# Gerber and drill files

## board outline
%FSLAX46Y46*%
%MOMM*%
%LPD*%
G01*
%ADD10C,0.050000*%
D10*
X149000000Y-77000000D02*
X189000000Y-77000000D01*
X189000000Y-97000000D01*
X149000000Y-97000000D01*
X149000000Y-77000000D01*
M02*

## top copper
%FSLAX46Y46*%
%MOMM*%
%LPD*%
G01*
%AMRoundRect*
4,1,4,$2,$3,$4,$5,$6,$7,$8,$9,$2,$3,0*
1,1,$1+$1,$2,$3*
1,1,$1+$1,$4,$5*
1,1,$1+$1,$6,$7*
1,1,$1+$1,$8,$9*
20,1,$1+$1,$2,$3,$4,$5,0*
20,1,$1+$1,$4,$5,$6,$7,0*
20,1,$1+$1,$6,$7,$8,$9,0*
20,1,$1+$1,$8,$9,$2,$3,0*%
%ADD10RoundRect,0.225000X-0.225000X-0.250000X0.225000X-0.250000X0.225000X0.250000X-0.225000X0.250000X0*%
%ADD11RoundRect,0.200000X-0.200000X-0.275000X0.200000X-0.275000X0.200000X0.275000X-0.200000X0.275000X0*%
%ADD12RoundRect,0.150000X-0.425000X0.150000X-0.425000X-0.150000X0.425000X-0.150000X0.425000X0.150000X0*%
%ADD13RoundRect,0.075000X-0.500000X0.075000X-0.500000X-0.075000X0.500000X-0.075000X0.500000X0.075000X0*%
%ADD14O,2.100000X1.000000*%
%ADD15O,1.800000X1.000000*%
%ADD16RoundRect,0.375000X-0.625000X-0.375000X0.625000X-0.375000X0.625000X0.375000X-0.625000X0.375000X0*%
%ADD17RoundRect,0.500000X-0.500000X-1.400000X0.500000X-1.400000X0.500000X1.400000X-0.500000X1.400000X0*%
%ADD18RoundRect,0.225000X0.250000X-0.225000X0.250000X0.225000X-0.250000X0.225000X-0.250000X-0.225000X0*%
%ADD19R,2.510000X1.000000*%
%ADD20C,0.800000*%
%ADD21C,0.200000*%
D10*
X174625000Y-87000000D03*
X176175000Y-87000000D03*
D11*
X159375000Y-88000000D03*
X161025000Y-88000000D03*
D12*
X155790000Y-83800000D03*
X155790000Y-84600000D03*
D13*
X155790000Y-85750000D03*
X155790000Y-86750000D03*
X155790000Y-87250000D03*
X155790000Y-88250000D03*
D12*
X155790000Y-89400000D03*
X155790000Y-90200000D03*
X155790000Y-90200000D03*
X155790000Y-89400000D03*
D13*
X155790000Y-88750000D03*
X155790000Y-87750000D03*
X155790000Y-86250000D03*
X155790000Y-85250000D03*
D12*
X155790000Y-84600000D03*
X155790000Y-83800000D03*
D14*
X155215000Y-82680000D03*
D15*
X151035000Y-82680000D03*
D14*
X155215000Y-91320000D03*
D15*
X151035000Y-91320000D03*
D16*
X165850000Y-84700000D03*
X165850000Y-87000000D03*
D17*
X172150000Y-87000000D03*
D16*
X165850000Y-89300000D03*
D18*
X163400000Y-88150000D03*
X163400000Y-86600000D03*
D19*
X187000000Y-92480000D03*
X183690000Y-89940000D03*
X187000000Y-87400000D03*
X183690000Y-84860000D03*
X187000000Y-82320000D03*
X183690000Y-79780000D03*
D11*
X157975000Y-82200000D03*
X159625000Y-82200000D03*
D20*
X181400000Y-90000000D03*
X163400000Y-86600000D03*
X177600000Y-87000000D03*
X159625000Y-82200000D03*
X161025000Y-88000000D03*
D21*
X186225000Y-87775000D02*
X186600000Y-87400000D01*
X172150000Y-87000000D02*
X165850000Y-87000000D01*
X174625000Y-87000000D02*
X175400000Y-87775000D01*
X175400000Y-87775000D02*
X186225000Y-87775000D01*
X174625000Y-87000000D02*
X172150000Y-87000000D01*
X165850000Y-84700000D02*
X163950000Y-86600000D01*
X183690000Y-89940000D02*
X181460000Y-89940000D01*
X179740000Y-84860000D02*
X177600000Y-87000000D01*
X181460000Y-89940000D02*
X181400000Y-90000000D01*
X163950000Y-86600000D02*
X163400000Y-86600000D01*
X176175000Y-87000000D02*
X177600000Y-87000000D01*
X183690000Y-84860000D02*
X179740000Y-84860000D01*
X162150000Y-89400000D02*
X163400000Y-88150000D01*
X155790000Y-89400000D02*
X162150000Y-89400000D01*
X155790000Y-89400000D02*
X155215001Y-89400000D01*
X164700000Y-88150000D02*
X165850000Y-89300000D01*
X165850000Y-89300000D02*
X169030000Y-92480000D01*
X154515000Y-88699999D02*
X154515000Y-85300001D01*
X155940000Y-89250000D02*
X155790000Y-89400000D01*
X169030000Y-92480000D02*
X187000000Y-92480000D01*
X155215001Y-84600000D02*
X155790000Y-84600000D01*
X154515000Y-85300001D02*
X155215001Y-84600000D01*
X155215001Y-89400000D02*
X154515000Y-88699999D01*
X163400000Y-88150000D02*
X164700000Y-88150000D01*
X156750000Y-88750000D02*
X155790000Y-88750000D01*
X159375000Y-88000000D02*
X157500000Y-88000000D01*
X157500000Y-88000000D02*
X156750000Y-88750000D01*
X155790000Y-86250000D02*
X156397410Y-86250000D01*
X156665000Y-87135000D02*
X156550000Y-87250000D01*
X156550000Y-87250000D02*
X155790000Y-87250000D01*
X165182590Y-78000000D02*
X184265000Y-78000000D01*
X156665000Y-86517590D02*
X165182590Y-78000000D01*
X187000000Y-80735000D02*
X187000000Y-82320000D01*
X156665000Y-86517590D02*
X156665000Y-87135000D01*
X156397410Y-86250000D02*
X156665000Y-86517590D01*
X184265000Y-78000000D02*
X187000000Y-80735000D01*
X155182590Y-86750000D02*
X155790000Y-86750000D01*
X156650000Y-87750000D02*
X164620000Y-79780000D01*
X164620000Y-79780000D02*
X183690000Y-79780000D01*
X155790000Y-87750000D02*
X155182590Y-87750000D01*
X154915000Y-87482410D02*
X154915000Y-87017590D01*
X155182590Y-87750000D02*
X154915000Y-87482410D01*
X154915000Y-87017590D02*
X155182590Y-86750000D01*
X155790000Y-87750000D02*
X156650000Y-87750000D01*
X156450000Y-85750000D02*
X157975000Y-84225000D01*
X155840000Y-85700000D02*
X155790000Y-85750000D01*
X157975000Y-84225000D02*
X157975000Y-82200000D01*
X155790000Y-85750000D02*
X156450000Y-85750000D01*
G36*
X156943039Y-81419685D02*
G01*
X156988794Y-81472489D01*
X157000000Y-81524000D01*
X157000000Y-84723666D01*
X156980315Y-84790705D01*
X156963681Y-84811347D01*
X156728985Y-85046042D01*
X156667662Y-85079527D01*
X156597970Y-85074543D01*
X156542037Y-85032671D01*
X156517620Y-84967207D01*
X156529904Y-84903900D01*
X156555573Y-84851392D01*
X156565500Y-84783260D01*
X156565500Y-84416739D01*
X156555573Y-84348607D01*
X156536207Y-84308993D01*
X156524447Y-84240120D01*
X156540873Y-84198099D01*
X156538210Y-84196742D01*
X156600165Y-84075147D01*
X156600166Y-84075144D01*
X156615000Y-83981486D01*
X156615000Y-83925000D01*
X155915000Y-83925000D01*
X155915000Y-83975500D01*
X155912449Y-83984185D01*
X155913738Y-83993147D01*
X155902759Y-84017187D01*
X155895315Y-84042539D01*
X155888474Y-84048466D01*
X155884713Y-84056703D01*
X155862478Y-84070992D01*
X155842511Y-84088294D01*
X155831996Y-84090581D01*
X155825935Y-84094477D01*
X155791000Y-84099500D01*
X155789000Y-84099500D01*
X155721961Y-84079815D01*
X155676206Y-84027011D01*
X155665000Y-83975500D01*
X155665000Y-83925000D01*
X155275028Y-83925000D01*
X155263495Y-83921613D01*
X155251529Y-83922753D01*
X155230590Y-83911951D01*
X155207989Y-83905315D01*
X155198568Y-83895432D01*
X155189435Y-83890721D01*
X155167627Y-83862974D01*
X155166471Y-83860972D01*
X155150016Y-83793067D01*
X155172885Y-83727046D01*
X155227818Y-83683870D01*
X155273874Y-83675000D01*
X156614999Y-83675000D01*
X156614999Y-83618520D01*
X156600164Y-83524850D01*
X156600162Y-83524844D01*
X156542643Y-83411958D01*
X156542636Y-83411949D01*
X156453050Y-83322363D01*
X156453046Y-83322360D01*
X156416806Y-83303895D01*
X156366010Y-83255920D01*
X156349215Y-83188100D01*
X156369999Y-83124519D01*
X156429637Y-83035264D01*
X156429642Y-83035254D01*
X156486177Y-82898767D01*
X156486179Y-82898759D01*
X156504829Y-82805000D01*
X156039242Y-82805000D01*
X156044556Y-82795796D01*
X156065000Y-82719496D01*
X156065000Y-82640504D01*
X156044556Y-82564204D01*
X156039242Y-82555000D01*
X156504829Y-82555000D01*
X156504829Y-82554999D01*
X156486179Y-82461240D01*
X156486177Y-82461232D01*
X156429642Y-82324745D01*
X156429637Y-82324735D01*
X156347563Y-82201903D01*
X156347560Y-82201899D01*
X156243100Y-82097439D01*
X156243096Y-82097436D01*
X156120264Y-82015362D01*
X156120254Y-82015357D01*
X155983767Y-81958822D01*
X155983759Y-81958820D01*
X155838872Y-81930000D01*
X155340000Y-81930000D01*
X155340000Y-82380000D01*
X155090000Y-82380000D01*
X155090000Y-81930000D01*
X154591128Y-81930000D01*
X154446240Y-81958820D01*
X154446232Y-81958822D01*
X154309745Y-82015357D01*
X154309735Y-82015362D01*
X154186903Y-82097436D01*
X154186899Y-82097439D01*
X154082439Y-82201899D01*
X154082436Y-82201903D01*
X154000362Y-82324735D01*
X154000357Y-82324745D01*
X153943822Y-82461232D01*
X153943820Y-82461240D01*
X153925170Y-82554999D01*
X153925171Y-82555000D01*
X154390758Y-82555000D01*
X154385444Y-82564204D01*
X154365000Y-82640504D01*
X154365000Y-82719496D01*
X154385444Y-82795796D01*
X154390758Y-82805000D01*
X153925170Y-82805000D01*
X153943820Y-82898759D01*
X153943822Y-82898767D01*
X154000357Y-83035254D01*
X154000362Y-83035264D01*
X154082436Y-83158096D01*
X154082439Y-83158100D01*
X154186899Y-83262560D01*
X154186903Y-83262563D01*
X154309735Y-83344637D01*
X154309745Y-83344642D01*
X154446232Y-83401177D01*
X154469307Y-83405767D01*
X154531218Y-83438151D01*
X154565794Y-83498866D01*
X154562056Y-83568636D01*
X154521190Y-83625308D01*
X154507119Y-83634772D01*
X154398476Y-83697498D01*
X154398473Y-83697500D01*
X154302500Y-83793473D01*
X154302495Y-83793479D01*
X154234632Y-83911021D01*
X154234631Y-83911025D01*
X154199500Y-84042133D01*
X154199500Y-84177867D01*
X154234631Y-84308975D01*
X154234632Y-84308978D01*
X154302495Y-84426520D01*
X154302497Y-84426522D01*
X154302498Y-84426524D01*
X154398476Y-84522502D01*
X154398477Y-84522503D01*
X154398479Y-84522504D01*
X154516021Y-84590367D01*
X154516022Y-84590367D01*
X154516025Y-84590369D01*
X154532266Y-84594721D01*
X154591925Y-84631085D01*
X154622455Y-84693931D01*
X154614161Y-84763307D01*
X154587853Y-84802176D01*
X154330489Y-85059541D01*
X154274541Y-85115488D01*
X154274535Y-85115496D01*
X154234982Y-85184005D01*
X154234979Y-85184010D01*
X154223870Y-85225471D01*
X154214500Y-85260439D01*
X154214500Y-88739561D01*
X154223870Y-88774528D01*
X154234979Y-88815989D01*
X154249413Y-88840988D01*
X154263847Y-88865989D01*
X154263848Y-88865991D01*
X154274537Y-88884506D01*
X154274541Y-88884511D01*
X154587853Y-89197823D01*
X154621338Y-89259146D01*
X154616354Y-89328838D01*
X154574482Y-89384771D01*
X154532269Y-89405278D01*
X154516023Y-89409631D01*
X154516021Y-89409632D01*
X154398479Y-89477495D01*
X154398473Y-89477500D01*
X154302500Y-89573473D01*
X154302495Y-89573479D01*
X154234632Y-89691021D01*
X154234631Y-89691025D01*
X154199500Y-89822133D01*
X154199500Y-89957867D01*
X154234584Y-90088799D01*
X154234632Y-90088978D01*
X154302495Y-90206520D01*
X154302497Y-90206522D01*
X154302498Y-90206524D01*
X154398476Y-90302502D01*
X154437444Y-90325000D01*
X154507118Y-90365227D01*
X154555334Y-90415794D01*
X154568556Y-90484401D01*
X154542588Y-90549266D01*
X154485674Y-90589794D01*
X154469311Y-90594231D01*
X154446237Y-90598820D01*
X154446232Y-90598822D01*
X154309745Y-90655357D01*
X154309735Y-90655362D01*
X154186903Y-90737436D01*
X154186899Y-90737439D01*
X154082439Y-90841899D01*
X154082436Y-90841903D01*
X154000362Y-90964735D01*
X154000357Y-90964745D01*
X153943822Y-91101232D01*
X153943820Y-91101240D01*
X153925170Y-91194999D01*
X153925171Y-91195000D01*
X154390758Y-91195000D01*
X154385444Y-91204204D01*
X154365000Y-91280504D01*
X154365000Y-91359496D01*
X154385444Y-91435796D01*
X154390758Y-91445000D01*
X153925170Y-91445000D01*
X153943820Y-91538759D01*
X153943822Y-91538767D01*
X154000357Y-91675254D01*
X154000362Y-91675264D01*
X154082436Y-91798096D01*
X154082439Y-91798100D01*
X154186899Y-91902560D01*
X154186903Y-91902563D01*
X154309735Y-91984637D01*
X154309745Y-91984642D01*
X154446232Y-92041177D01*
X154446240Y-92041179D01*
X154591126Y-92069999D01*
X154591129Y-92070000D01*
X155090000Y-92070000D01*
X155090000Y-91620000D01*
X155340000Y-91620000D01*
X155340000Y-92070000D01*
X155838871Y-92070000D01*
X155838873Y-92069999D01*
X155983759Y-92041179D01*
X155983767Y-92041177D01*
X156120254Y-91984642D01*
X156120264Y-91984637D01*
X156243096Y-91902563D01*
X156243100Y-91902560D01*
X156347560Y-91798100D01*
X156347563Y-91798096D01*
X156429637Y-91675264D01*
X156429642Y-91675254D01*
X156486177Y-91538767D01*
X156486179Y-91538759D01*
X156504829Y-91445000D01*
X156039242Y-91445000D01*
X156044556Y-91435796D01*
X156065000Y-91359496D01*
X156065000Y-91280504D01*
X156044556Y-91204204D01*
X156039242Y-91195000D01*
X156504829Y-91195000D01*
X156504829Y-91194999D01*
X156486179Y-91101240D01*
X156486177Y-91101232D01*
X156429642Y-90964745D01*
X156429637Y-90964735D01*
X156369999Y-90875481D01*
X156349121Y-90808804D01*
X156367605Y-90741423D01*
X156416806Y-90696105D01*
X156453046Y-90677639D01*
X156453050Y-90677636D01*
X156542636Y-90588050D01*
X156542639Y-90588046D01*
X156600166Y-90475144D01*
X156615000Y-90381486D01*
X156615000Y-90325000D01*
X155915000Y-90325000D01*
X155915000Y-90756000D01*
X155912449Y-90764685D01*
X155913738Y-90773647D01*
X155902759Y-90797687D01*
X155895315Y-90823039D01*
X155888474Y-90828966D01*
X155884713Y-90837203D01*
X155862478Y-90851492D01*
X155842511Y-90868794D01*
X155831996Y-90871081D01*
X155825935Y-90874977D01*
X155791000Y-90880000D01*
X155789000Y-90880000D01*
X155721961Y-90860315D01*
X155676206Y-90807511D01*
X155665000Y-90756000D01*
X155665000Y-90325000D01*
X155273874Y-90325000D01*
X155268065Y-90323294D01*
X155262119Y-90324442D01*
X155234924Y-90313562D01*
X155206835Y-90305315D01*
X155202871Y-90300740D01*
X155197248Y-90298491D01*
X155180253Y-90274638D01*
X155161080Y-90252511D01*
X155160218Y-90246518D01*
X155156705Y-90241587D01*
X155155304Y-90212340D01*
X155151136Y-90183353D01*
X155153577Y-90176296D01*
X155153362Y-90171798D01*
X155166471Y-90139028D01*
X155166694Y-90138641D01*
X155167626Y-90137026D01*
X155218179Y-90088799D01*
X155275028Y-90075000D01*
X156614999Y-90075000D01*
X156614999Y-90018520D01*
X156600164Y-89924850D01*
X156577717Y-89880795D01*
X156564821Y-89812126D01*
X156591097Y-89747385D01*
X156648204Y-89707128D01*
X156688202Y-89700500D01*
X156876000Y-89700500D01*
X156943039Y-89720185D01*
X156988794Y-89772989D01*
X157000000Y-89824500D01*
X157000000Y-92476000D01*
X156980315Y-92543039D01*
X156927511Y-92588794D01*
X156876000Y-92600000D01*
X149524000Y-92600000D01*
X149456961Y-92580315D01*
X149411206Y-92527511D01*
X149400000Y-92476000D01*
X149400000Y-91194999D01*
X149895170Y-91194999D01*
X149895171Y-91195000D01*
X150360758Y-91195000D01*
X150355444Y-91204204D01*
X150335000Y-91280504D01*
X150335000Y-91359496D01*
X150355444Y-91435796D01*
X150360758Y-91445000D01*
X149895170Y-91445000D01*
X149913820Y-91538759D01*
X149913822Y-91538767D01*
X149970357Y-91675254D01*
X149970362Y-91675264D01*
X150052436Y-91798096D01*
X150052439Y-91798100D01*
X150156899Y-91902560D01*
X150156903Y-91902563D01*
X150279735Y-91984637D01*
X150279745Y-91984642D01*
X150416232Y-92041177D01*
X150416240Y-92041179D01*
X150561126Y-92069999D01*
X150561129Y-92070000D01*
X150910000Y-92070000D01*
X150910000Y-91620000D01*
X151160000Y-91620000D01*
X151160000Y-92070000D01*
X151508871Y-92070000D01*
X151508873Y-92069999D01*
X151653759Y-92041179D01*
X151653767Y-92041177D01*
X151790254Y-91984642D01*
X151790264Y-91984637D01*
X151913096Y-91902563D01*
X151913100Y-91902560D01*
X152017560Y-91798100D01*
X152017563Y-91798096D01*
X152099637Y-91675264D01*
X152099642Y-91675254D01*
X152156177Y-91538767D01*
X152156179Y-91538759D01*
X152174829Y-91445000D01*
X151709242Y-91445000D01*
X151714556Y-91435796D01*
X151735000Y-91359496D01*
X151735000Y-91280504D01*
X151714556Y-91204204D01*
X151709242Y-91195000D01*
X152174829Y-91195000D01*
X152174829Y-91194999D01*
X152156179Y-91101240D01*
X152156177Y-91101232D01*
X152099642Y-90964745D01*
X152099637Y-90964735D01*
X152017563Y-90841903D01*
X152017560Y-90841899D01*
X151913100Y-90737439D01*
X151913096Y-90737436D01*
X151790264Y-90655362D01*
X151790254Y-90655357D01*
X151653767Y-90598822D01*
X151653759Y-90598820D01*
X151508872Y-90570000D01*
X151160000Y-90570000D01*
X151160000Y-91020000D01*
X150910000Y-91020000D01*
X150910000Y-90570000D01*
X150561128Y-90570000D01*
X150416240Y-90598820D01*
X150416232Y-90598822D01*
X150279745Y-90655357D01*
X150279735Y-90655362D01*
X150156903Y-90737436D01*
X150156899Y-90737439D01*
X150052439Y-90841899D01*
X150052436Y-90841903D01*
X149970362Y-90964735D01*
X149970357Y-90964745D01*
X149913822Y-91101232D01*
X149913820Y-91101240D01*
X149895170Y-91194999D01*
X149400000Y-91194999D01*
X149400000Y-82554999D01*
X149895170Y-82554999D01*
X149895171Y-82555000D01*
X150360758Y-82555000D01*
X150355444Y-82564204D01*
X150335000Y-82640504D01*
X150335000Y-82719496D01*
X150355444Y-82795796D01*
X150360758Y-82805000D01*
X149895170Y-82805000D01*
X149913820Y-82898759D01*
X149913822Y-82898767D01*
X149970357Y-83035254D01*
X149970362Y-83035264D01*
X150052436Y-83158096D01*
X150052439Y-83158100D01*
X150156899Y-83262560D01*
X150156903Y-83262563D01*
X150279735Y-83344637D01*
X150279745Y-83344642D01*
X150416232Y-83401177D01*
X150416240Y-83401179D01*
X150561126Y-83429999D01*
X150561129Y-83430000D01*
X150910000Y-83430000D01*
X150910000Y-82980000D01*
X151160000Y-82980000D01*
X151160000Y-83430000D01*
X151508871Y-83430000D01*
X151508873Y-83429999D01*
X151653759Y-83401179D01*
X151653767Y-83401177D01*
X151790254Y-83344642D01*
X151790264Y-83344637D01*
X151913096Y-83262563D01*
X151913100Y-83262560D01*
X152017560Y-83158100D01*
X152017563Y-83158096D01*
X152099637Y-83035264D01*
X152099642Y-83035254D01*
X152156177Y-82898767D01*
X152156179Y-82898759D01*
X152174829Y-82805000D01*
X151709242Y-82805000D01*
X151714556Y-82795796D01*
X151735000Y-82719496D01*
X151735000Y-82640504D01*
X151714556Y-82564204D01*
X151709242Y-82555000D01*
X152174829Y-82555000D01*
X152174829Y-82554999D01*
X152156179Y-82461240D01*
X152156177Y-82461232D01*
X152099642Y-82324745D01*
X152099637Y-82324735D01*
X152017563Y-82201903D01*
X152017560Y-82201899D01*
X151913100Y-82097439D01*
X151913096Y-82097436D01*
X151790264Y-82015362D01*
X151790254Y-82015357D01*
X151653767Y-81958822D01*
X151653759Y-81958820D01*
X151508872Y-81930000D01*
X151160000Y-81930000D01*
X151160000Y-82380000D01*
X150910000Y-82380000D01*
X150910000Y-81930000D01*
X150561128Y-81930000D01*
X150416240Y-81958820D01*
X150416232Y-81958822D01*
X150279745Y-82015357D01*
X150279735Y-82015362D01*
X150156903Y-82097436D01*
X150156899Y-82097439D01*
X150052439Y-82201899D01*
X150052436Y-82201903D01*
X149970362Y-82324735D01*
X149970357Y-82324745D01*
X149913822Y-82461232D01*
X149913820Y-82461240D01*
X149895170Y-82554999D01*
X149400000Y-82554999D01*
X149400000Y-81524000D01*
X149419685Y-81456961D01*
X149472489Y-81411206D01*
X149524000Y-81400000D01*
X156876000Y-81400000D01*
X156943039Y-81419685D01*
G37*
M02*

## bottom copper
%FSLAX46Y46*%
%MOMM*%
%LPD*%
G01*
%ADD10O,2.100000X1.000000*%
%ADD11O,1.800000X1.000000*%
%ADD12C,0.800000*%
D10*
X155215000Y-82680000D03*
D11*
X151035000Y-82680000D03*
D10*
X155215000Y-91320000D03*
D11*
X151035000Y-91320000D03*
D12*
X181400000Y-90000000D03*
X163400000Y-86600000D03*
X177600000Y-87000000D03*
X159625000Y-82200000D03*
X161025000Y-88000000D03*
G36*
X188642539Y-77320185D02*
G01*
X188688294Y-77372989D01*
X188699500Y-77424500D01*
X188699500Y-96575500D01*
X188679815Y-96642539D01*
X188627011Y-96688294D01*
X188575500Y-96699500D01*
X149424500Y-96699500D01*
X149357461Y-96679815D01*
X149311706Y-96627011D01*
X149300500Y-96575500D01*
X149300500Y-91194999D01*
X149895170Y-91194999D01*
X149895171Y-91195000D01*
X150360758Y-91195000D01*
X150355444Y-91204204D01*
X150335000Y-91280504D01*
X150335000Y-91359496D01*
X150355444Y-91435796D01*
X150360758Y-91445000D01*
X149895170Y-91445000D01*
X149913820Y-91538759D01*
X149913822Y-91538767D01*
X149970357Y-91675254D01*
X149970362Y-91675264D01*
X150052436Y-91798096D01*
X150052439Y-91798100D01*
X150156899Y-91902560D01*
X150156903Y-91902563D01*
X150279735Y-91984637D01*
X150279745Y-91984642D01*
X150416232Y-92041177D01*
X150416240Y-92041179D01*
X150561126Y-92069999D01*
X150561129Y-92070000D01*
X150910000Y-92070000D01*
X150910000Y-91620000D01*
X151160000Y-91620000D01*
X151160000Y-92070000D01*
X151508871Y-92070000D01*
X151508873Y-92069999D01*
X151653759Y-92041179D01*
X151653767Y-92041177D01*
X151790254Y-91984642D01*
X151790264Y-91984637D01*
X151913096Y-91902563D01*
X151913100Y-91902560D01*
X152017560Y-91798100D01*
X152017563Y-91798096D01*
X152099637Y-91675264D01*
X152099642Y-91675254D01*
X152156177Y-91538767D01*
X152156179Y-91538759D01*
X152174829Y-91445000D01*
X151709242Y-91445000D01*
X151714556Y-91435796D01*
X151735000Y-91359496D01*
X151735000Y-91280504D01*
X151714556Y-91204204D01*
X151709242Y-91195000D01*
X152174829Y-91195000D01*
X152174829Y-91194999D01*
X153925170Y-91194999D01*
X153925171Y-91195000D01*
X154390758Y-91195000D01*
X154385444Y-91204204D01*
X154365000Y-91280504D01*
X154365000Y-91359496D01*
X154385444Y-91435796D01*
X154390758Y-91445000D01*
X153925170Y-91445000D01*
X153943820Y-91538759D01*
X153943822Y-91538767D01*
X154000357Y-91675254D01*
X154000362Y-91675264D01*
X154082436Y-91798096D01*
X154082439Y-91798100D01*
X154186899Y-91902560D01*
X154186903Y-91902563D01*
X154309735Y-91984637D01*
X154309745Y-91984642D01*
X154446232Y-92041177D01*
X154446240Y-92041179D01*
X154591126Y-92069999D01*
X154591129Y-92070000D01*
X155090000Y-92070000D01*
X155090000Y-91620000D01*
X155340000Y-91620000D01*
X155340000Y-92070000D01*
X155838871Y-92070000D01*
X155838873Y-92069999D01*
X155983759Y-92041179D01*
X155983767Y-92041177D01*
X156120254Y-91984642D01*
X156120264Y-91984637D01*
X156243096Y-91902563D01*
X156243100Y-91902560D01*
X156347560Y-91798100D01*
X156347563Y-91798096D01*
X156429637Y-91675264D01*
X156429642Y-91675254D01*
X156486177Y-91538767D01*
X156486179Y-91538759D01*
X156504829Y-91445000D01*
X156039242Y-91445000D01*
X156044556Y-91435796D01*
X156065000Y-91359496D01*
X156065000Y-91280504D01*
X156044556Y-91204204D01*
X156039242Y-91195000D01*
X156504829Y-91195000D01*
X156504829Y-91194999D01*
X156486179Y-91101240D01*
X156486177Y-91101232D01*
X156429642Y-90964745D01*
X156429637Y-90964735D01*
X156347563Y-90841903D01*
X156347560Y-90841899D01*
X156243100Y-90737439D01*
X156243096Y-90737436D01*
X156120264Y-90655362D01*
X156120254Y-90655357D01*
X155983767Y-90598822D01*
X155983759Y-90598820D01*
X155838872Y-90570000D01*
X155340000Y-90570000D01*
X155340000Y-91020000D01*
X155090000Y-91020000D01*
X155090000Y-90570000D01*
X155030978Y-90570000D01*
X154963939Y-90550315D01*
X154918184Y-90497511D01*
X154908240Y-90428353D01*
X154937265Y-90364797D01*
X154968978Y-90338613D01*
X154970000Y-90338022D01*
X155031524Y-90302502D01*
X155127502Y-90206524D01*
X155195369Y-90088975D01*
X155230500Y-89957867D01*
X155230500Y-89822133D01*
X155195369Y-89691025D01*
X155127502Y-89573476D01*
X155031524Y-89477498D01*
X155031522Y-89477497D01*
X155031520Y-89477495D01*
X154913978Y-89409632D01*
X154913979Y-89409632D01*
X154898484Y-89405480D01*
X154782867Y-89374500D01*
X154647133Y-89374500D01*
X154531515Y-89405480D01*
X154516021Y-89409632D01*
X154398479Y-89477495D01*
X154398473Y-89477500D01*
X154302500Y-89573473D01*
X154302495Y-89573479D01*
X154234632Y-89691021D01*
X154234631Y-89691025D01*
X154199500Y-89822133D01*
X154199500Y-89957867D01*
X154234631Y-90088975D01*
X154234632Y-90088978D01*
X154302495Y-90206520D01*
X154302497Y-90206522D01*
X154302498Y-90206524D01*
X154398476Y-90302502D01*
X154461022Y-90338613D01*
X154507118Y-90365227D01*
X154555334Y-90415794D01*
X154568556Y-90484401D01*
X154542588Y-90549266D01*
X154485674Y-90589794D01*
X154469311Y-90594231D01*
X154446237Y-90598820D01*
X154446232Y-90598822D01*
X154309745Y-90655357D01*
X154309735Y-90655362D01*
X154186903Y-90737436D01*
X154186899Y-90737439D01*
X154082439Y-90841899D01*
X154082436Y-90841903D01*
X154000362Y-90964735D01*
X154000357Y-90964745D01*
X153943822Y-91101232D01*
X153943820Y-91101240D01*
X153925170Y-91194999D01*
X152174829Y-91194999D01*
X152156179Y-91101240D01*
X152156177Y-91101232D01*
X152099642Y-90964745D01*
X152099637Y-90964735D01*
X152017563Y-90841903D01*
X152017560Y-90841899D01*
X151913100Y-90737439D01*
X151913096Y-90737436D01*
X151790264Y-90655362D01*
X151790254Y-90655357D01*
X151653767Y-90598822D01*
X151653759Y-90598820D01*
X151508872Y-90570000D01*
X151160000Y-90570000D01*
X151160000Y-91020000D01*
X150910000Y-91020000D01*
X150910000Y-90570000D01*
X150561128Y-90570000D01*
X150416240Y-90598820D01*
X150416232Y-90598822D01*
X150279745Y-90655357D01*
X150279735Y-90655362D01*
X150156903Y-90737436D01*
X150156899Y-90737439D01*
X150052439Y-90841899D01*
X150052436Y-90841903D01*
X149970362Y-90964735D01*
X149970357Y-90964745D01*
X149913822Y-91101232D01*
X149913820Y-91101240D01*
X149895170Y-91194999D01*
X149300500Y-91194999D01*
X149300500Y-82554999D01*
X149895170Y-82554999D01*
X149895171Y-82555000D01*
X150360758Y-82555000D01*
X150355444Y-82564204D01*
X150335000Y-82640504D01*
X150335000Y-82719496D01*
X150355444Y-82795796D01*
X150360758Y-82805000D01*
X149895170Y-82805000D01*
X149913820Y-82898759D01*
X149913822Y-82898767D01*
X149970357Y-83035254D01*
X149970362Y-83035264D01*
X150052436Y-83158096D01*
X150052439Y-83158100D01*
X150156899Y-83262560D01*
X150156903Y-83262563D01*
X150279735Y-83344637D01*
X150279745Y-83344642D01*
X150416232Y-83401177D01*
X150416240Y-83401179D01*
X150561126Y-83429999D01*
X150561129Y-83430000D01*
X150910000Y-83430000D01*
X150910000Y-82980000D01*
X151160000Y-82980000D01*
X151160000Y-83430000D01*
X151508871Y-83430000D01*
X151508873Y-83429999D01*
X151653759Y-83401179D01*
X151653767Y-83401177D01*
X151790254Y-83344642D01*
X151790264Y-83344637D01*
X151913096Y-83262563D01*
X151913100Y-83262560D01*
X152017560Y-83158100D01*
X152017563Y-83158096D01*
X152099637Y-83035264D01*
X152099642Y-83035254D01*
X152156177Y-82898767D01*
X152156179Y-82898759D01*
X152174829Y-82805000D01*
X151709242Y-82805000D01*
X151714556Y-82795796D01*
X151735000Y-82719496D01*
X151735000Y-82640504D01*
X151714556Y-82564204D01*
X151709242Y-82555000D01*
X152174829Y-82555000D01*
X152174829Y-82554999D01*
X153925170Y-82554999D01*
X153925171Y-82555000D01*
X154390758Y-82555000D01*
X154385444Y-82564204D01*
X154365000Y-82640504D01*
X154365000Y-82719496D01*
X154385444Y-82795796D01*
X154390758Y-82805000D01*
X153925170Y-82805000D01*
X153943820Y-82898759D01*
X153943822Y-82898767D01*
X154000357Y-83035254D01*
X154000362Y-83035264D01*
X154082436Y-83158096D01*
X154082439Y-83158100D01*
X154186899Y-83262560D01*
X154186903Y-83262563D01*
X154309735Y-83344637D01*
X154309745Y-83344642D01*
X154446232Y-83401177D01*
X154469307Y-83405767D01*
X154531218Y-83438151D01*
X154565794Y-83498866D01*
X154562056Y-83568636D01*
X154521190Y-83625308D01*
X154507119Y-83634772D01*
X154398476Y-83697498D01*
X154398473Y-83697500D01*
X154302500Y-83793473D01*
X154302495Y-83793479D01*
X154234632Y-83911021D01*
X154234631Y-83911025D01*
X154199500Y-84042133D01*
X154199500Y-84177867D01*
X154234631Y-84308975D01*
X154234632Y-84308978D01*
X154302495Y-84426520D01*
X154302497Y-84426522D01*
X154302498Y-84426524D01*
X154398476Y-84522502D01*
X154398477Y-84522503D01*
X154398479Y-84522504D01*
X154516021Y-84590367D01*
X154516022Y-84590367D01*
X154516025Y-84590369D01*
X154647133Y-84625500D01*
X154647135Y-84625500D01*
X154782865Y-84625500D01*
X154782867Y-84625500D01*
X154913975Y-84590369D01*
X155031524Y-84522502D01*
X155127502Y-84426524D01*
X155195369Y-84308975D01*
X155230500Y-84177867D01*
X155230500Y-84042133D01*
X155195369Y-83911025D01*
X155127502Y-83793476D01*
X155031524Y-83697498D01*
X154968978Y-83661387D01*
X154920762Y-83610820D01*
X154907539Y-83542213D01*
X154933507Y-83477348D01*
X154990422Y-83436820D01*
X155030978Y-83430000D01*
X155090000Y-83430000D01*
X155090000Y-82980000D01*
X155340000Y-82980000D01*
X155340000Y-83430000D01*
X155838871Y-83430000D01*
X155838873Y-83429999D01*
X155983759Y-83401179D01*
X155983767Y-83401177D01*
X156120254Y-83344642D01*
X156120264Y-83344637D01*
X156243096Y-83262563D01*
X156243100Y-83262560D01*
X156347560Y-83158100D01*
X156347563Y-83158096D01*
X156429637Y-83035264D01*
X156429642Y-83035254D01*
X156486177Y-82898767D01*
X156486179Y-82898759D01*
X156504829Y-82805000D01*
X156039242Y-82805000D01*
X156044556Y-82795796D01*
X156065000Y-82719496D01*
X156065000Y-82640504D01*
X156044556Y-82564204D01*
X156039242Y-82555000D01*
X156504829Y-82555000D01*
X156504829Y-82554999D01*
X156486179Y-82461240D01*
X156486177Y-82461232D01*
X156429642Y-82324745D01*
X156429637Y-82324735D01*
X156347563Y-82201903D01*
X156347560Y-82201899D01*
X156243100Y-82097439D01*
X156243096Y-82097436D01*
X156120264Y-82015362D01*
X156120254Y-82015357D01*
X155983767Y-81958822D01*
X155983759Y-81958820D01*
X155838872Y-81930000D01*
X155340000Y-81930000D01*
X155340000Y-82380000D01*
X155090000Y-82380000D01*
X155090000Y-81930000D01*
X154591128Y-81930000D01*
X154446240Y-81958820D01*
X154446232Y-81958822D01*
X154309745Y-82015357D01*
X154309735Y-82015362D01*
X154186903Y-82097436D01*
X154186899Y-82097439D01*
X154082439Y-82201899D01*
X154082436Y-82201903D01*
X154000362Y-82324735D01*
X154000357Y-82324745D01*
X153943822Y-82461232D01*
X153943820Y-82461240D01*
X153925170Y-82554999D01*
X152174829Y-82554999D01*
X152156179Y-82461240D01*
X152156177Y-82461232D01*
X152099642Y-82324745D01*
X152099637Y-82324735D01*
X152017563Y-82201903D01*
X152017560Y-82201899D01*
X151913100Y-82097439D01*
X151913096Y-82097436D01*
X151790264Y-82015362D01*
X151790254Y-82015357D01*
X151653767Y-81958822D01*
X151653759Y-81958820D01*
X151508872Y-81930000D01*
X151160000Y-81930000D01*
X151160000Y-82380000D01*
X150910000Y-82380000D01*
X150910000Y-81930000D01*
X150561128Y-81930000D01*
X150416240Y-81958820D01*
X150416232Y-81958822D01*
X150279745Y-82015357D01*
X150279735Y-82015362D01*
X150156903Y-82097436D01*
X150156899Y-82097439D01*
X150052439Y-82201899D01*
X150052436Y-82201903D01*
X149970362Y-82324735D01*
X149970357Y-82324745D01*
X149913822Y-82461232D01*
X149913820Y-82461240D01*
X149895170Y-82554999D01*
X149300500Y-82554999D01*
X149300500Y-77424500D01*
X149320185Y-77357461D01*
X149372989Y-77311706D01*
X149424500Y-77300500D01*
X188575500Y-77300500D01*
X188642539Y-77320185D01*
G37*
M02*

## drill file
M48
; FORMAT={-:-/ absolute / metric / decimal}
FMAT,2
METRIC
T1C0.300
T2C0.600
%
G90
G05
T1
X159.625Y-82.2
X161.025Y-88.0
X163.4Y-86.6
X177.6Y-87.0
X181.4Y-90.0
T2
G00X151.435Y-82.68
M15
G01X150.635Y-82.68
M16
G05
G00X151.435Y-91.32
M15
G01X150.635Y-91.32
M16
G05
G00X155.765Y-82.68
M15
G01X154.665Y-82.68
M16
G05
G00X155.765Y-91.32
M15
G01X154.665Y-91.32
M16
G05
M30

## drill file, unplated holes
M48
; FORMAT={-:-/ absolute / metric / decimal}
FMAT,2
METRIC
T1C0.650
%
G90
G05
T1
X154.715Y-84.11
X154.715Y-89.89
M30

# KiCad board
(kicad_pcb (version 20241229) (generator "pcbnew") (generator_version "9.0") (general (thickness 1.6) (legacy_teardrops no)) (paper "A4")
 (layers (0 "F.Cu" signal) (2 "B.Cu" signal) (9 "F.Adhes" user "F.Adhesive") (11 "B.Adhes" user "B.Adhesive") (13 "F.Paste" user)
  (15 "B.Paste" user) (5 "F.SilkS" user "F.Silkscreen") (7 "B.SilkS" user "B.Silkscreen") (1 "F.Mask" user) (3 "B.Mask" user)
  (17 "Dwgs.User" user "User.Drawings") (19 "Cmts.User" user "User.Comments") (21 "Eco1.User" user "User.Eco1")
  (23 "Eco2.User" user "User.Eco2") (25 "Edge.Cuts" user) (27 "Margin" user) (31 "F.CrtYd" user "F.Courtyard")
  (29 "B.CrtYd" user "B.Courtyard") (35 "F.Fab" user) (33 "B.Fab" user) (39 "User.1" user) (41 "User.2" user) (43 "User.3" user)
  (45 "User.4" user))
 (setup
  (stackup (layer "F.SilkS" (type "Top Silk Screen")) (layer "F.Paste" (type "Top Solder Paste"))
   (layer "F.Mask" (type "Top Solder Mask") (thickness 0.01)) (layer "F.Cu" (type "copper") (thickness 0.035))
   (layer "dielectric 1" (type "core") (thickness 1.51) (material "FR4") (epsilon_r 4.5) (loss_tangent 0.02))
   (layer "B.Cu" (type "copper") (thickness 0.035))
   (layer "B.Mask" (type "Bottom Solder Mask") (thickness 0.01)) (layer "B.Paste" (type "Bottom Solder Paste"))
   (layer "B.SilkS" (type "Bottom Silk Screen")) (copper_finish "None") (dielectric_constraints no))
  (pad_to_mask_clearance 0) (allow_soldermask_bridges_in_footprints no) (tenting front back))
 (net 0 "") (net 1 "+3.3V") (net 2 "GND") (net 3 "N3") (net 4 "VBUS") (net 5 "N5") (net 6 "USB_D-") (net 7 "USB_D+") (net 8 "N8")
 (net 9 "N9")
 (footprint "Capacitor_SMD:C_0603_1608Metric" (layer "F.Cu") (at 175.4 87)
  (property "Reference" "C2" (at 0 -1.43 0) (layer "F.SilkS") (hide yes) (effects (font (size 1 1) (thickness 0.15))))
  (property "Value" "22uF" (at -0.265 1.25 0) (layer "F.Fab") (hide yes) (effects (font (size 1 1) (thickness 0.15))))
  (pad "1" smd roundrect (at -0.775 0) (size 0.9 0.95) (layers "F.Cu" "F.Mask" "F.Paste") (roundrect_rratio 0.25) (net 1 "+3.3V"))
  (pad "2" smd roundrect (at 0.775 0) (size 0.9 0.95) (layers "F.Cu" "F.Mask" "F.Paste") (roundrect_rratio 0.25) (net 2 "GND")))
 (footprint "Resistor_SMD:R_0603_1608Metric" (layer "F.Cu") (at 160.2 88)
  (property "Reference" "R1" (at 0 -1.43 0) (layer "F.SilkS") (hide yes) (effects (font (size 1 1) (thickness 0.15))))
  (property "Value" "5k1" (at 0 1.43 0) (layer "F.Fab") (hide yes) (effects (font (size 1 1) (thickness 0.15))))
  (pad "1" smd roundrect (at -0.825 0) (size 0.8 0.95) (layers "F.Cu" "F.Mask" "F.Paste") (roundrect_rratio 0.25) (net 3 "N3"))
  (pad "2" smd roundrect (at 0.825 0) (size 0.8 0.95) (layers "F.Cu" "F.Mask" "F.Paste") (roundrect_rratio 0.25) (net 2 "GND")))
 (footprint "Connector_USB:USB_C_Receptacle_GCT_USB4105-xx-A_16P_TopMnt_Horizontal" (layer "F.Cu") (at 152.11 87 -90)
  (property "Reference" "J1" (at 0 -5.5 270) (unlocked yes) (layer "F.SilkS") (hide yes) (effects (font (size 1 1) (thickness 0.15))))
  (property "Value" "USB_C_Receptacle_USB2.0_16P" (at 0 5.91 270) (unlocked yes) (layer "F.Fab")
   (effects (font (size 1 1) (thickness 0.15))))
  (pad "" np_thru_hole circle (at -2.89 -2.605 270) (size 0.65 0.65) (drill 0.65) (layers "*.Cu" "*.Mask"))
  (pad "" np_thru_hole circle (at 2.89 -2.605 270) (size 0.65 0.65) (drill 0.65) (layers "*.Cu" "*.Mask"))
  (pad "A1" smd roundrect (at -3.2 -3.68 270) (size 0.6 1.15) (layers "F.Cu" "F.Mask" "F.Paste") (roundrect_rratio 0.25) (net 2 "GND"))
  (pad "A4" smd roundrect (at -2.4 -3.68 270) (size 0.6 1.15) (layers "F.Cu" "F.Mask" "F.Paste") (roundrect_rratio 0.25) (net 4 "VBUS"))
  (pad "A5" smd roundrect (at -1.25 -3.68 270) (size 0.3 1.15) (layers "F.Cu" "F.Mask" "F.Paste") (roundrect_rratio 0.25) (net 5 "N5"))
  (pad "A6" smd roundrect (at -0.25 -3.68 270) (size 0.3 1.15) (layers "F.Cu" "F.Mask" "F.Paste") (roundrect_rratio 0.25) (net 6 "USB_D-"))
  (pad "A7" smd roundrect (at 0.25 -3.68 270) (size 0.3 1.15) (layers "F.Cu" "F.Mask" "F.Paste") (roundrect_rratio 0.25) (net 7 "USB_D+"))
  (pad "A8" smd roundrect (at 1.25 -3.68 270) (size 0.3 1.15) (layers "F.Cu" "F.Mask" "F.Paste") (roundrect_rratio 0.25) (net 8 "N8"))
  (pad "A9" smd roundrect (at 2.4 -3.68 270) (size 0.6 1.15) (layers "F.Cu" "F.Mask" "F.Paste") (roundrect_rratio 0.25) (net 4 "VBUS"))
  (pad "A12" smd roundrect (at 3.2 -3.68 270) (size 0.6 1.15) (layers "F.Cu" "F.Mask" "F.Paste") (roundrect_rratio 0.25) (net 2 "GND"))
  (pad "B1" smd roundrect (at 3.2 -3.68 270) (size 0.6 1.15) (layers "F.Cu" "F.Mask" "F.Paste") (roundrect_rratio 0.25) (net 2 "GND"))
  (pad "B4" smd roundrect (at 2.4 -3.68 270) (size 0.6 1.15) (layers "F.Cu" "F.Mask" "F.Paste") (roundrect_rratio 0.25) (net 4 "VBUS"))
  (pad "B5" smd roundrect (at 1.75 -3.68 270) (size 0.3 1.15) (layers "F.Cu" "F.Mask" "F.Paste") (roundrect_rratio 0.25) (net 3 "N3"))
  (pad "B6" smd roundrect (at 0.75 -3.68 270) (size 0.3 1.15) (layers "F.Cu" "F.Mask" "F.Paste") (roundrect_rratio 0.25) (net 6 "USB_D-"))
  (pad "B7" smd roundrect (at -0.75 -3.68 270) (size 0.3 1.15) (layers "F.Cu" "F.Mask" "F.Paste") (roundrect_rratio 0.25) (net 7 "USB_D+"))
  (pad "B8" smd roundrect (at -1.75 -3.68 270) (size 0.3 1.15) (layers "F.Cu" "F.Mask" "F.Paste") (roundrect_rratio 0.25) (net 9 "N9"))
  (pad "B9" smd roundrect (at -2.4 -3.68 270) (size 0.6 1.15) (layers "F.Cu" "F.Mask" "F.Paste") (roundrect_rratio 0.25) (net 4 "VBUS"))
  (pad "B12" smd roundrect (at -3.2 -3.68 270) (size 0.6 1.15) (layers "F.Cu" "F.Mask" "F.Paste") (roundrect_rratio 0.25) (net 2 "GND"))
  (pad "S1" thru_hole oval (at -4.32 -3.105 270) (size 1 2.1) (drill oval 0.6 1.7) (layers "*.Cu" "*.Mask" "F.Paste")
   (remove_unused_layers no) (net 2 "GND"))
  (pad "S1" thru_hole oval (at -4.32 1.075 270) (size 1 1.8) (drill oval 0.6 1.4) (layers "*.Cu" "*.Mask" "F.Paste")
   (remove_unused_layers no) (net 2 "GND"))
  (pad "S1" thru_hole oval (at 4.32 -3.105 270) (size 1 2.1) (drill oval 0.6 1.7) (layers "*.Cu" "*.Mask" "F.Paste")
   (remove_unused_layers no) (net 2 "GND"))
  (pad "S1" thru_hole oval (at 4.32 1.075 270) (size 1 1.8) (drill oval 0.6 1.4) (layers "*.Cu" "*.Mask" "F.Paste")
   (remove_unused_layers no) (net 2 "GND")))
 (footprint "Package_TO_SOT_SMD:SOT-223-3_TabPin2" (layer "F.Cu") (at 169 87)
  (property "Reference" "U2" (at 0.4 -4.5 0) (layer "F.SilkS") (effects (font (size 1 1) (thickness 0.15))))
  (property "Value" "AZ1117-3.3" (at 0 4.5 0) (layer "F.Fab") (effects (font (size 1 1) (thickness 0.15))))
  (pad "1" smd roundrect (at -3.15 -2.3) (size 2 1.5) (layers "F.Cu" "F.Mask" "F.Paste") (roundrect_rratio 0.25) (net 2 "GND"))
  (pad "2" smd roundrect (at -3.15 0) (size 2 1.5) (layers "F.Cu" "F.Mask" "F.Paste") (roundrect_rratio 0.25) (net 1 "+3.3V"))
  (pad "2" smd roundrect (at 3.15 0) (size 2 3.8) (layers "F.Cu" "F.Mask" "F.Paste") (roundrect_rratio 0.25) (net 1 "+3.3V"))
  (pad "3" smd roundrect (at -3.15 2.3) (size 2 1.5) (layers "F.Cu" "F.Mask" "F.Paste") (roundrect_rratio 0.25) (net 4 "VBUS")))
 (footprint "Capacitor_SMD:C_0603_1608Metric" (layer "F.Cu") (at 163.4 87.375 90)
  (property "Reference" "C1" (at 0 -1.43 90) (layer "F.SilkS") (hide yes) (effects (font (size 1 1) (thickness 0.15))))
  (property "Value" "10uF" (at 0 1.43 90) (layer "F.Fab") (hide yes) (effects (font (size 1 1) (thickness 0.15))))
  (pad "1" smd roundrect (at -0.775 0 90) (size 0.9 0.95) (layers "F.Cu" "F.Mask" "F.Paste") (roundrect_rratio 0.25) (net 4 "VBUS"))
  (pad "2" smd roundrect (at 0.775 0 90) (size 0.9 0.95) (layers "F.Cu" "F.Mask" "F.Paste") (roundrect_rratio 0.25) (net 2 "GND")))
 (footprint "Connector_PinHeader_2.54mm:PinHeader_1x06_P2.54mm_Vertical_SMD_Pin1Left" (layer "F.Cu") (at 185.345 86.13 180)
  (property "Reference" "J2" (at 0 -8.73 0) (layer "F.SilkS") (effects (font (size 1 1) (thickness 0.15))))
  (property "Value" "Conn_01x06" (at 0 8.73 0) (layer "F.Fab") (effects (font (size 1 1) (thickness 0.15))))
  (pad "1" smd rect (at -1.655 -6.35 180) (size 2.51 1) (layers "F.Cu" "F.Mask" "F.Paste") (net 4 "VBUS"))
  (pad "2" smd rect (at 1.655 -3.81 180) (size 2.51 1) (layers "F.Cu" "F.Mask" "F.Paste") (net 2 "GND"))
  (pad "3" smd rect (at -1.655 -1.27 180) (size 2.51 1) (layers "F.Cu" "F.Mask" "F.Paste") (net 1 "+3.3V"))
  (pad "4" smd rect (at 1.655 1.27 180) (size 2.51 1) (layers "F.Cu" "F.Mask" "F.Paste") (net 2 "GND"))
  (pad "5" smd rect (at -1.655 3.81 180) (size 2.51 1) (layers "F.Cu" "F.Mask" "F.Paste") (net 7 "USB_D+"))
  (pad "6" smd rect (at 1.655 6.35 180) (size 2.51 1) (layers "F.Cu" "F.Mask" "F.Paste") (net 6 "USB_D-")))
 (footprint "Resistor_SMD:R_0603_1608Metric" (layer "F.Cu") (at 158.8 82.2)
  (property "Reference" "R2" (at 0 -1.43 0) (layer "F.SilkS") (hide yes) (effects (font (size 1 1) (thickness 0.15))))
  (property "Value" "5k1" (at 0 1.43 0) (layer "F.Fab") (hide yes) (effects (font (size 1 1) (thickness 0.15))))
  (pad "1" smd roundrect (at -0.825 0) (size 0.8 0.95) (layers "F.Cu" "F.Mask" "F.Paste") (roundrect_rratio 0.25) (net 5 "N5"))
  (pad "2" smd roundrect (at 0.825 0) (size 0.8 0.95) (layers "F.Cu" "F.Mask" "F.Paste") (roundrect_rratio 0.25) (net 2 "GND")))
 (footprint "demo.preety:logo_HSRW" (layer "F.Cu") (at 161.4 94)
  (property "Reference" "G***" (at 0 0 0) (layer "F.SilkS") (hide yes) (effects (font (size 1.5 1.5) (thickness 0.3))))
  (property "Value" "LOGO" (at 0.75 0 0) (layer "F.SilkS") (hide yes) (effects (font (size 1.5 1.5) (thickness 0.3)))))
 (gr_rect (start 149 77) (end 189 97) (stroke (width 0.05) (type default)) (fill no) (layer "Edge.Cuts"))
 (segment (start 186.225 87.775) (end 186.6 87.4) (width 0.2) (layer "F.Cu") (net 1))
 (segment (start 172.15 87) (end 165.85 87) (width 0.2) (layer "F.Cu") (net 1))
 (segment (start 174.625 87) (end 175.4 87.775) (width 0.2) (layer "F.Cu") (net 1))
 (segment (start 175.4 87.775) (end 186.225 87.775) (width 0.2) (layer "F.Cu") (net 1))
 (segment (start 174.625 87) (end 172.15 87) (width 0.2) (layer "F.Cu") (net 1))
 (segment (start 165.85 84.7) (end 163.95 86.6) (width 0.2) (layer "F.Cu") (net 2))
 (segment (start 183.69 89.94) (end 181.46 89.94) (width 0.2) (layer "F.Cu") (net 2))
 (segment (start 179.74 84.86) (end 177.6 87) (width 0.2) (layer "F.Cu") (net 2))
 (segment (start 181.46 89.94) (end 181.4 90) (width 0.2) (layer "F.Cu") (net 2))
 (segment (start 163.95 86.6) (end 163.4 86.6) (width 0.2) (layer "F.Cu") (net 2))
 (segment (start 176.175 87) (end 177.6 87) (width 0.2) (layer "F.Cu") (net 2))
 (segment (start 183.69 84.86) (end 179.74 84.86) (width 0.2) (layer "F.Cu") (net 2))
 (via (at 181.4 90) (size 0.8) (drill 0.3) (layers "F.Cu" "B.Cu") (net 2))
 (via (at 163.4 86.6) (size 0.8) (drill 0.3) (layers "F.Cu" "B.Cu") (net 2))
 (via (at 177.6 87) (size 0.8) (drill 0.3) (layers "F.Cu" "B.Cu") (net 2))
 (via (at 159.625 82.2) (size 0.8) (drill 0.3) (layers "F.Cu" "B.Cu") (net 2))
 (via (at 161.025 88) (size 0.8) (drill 0.3) (layers "F.Cu" "B.Cu") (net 2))
 (segment (start 162.15 89.4) (end 163.4 88.15) (width 0.2) (layer "F.Cu") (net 4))
 (segment (start 155.79 89.4) (end 162.15 89.4) (width 0.2) (layer "F.Cu") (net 4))
 (segment (start 155.79 89.4) (end 155.215001 89.4) (width 0.2) (layer "F.Cu") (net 4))
 (segment (start 164.7 88.15) (end 165.85 89.3) (width 0.2) (layer "F.Cu") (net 4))
 (segment (start 165.85 89.3) (end 169.03 92.48) (width 0.2) (layer "F.Cu") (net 4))
 (segment (start 154.515 88.699999) (end 154.515 85.300001) (width 0.2) (layer "F.Cu") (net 4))
 (segment (start 155.94 89.25) (end 155.79 89.4) (width 0.2) (layer "F.Cu") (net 4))
 (segment (start 169.03 92.48) (end 187 92.48) (width 0.2) (layer "F.Cu") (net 4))
 (segment (start 155.215001 84.6) (end 155.79 84.6) (width 0.2) (layer "F.Cu") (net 4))
 (segment (start 154.515 85.300001) (end 155.215001 84.6) (width 0.2) (layer "F.Cu") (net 4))
 (segment (start 155.215001 89.4) (end 154.515 88.699999) (width 0.2) (layer "F.Cu") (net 4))
 (segment (start 163.4 88.15) (end 164.7 88.15) (width 0.2) (layer "F.Cu") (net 4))
 (segment (start 156.75 88.75) (end 155.79 88.75) (width 0.2) (layer "F.Cu") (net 3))
 (segment (start 159.375 88) (end 157.5 88) (width 0.2) (layer "F.Cu") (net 3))
 (segment (start 157.5 88) (end 156.75 88.75) (width 0.2) (layer "F.Cu") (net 3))
 (segment (start 155.79 86.25) (end 156.39741 86.25) (width 0.2) (layer "F.Cu") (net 7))
 (segment (start 156.665 87.135) (end 156.55 87.25) (width 0.2) (layer "F.Cu") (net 7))
 (segment (start 156.55 87.25) (end 155.79 87.25) (width 0.2) (layer "F.Cu") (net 7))
 (segment (start 165.18259 78) (end 184.265 78) (width 0.2) (layer "F.Cu") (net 7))
 (segment (start 156.665 86.51759) (end 165.18259 78) (width 0.2) (layer "F.Cu") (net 7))
 (segment (start 187 80.735) (end 187 82.32) (width 0.2) (layer "F.Cu") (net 7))
 (segment (start 156.665 86.51759) (end 156.665 87.135) (width 0.2) (layer "F.Cu") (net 7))
 (segment (start 156.39741 86.25) (end 156.665 86.51759) (width 0.2) (layer "F.Cu") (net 7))
 (segment (start 184.265 78) (end 187 80.735) (width 0.2) (layer "F.Cu") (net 7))
 (segment (start 155.18259 86.75) (end 155.79 86.75) (width 0.2) (layer "F.Cu") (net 6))
 (segment (start 156.65 87.75) (end 164.62 79.78) (width 0.2) (layer "F.Cu") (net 6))
 (segment (start 164.62 79.78) (end 183.69 79.78) (width 0.2) (layer "F.Cu") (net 6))
 (segment (start 155.79 87.75) (end 155.18259 87.75) (width 0.2) (layer "F.Cu") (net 6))
 (segment (start 154.915 87.48241) (end 154.915 87.01759) (width 0.2) (layer "F.Cu") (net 6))
 (segment (start 155.18259 87.75) (end 154.915 87.48241) (width 0.2) (layer "F.Cu") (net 6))
 (segment (start 154.915 87.01759) (end 155.18259 86.75) (width 0.2) (layer "F.Cu") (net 6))
 (segment (start 155.79 87.75) (end 156.65 87.75) (width 0.2) (layer "F.Cu") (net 6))
 (segment (start 156.45 85.75) (end 157.975 84.225) (width 0.2) (layer "F.Cu") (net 5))
 (segment (start 155.84 85.7) (end 155.79 85.75) (width 0.2) (layer "F.Cu") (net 5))
 (segment (start 157.975 84.225) (end 157.975 82.2) (width 0.2) (layer "F.Cu") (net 5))
 (segment (start 155.79 85.75) (end 156.45 85.75) (width 0.2) (layer "F.Cu") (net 5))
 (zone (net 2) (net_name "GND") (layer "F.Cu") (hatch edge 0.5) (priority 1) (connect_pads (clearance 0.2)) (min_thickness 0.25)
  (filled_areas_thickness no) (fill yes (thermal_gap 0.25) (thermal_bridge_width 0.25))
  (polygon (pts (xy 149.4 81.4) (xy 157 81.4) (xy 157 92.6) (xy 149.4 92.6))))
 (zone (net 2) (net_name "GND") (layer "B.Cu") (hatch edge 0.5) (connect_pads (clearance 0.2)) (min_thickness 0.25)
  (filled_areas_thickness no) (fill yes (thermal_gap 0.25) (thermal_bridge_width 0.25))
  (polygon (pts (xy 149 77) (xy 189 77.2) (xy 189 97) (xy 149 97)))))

